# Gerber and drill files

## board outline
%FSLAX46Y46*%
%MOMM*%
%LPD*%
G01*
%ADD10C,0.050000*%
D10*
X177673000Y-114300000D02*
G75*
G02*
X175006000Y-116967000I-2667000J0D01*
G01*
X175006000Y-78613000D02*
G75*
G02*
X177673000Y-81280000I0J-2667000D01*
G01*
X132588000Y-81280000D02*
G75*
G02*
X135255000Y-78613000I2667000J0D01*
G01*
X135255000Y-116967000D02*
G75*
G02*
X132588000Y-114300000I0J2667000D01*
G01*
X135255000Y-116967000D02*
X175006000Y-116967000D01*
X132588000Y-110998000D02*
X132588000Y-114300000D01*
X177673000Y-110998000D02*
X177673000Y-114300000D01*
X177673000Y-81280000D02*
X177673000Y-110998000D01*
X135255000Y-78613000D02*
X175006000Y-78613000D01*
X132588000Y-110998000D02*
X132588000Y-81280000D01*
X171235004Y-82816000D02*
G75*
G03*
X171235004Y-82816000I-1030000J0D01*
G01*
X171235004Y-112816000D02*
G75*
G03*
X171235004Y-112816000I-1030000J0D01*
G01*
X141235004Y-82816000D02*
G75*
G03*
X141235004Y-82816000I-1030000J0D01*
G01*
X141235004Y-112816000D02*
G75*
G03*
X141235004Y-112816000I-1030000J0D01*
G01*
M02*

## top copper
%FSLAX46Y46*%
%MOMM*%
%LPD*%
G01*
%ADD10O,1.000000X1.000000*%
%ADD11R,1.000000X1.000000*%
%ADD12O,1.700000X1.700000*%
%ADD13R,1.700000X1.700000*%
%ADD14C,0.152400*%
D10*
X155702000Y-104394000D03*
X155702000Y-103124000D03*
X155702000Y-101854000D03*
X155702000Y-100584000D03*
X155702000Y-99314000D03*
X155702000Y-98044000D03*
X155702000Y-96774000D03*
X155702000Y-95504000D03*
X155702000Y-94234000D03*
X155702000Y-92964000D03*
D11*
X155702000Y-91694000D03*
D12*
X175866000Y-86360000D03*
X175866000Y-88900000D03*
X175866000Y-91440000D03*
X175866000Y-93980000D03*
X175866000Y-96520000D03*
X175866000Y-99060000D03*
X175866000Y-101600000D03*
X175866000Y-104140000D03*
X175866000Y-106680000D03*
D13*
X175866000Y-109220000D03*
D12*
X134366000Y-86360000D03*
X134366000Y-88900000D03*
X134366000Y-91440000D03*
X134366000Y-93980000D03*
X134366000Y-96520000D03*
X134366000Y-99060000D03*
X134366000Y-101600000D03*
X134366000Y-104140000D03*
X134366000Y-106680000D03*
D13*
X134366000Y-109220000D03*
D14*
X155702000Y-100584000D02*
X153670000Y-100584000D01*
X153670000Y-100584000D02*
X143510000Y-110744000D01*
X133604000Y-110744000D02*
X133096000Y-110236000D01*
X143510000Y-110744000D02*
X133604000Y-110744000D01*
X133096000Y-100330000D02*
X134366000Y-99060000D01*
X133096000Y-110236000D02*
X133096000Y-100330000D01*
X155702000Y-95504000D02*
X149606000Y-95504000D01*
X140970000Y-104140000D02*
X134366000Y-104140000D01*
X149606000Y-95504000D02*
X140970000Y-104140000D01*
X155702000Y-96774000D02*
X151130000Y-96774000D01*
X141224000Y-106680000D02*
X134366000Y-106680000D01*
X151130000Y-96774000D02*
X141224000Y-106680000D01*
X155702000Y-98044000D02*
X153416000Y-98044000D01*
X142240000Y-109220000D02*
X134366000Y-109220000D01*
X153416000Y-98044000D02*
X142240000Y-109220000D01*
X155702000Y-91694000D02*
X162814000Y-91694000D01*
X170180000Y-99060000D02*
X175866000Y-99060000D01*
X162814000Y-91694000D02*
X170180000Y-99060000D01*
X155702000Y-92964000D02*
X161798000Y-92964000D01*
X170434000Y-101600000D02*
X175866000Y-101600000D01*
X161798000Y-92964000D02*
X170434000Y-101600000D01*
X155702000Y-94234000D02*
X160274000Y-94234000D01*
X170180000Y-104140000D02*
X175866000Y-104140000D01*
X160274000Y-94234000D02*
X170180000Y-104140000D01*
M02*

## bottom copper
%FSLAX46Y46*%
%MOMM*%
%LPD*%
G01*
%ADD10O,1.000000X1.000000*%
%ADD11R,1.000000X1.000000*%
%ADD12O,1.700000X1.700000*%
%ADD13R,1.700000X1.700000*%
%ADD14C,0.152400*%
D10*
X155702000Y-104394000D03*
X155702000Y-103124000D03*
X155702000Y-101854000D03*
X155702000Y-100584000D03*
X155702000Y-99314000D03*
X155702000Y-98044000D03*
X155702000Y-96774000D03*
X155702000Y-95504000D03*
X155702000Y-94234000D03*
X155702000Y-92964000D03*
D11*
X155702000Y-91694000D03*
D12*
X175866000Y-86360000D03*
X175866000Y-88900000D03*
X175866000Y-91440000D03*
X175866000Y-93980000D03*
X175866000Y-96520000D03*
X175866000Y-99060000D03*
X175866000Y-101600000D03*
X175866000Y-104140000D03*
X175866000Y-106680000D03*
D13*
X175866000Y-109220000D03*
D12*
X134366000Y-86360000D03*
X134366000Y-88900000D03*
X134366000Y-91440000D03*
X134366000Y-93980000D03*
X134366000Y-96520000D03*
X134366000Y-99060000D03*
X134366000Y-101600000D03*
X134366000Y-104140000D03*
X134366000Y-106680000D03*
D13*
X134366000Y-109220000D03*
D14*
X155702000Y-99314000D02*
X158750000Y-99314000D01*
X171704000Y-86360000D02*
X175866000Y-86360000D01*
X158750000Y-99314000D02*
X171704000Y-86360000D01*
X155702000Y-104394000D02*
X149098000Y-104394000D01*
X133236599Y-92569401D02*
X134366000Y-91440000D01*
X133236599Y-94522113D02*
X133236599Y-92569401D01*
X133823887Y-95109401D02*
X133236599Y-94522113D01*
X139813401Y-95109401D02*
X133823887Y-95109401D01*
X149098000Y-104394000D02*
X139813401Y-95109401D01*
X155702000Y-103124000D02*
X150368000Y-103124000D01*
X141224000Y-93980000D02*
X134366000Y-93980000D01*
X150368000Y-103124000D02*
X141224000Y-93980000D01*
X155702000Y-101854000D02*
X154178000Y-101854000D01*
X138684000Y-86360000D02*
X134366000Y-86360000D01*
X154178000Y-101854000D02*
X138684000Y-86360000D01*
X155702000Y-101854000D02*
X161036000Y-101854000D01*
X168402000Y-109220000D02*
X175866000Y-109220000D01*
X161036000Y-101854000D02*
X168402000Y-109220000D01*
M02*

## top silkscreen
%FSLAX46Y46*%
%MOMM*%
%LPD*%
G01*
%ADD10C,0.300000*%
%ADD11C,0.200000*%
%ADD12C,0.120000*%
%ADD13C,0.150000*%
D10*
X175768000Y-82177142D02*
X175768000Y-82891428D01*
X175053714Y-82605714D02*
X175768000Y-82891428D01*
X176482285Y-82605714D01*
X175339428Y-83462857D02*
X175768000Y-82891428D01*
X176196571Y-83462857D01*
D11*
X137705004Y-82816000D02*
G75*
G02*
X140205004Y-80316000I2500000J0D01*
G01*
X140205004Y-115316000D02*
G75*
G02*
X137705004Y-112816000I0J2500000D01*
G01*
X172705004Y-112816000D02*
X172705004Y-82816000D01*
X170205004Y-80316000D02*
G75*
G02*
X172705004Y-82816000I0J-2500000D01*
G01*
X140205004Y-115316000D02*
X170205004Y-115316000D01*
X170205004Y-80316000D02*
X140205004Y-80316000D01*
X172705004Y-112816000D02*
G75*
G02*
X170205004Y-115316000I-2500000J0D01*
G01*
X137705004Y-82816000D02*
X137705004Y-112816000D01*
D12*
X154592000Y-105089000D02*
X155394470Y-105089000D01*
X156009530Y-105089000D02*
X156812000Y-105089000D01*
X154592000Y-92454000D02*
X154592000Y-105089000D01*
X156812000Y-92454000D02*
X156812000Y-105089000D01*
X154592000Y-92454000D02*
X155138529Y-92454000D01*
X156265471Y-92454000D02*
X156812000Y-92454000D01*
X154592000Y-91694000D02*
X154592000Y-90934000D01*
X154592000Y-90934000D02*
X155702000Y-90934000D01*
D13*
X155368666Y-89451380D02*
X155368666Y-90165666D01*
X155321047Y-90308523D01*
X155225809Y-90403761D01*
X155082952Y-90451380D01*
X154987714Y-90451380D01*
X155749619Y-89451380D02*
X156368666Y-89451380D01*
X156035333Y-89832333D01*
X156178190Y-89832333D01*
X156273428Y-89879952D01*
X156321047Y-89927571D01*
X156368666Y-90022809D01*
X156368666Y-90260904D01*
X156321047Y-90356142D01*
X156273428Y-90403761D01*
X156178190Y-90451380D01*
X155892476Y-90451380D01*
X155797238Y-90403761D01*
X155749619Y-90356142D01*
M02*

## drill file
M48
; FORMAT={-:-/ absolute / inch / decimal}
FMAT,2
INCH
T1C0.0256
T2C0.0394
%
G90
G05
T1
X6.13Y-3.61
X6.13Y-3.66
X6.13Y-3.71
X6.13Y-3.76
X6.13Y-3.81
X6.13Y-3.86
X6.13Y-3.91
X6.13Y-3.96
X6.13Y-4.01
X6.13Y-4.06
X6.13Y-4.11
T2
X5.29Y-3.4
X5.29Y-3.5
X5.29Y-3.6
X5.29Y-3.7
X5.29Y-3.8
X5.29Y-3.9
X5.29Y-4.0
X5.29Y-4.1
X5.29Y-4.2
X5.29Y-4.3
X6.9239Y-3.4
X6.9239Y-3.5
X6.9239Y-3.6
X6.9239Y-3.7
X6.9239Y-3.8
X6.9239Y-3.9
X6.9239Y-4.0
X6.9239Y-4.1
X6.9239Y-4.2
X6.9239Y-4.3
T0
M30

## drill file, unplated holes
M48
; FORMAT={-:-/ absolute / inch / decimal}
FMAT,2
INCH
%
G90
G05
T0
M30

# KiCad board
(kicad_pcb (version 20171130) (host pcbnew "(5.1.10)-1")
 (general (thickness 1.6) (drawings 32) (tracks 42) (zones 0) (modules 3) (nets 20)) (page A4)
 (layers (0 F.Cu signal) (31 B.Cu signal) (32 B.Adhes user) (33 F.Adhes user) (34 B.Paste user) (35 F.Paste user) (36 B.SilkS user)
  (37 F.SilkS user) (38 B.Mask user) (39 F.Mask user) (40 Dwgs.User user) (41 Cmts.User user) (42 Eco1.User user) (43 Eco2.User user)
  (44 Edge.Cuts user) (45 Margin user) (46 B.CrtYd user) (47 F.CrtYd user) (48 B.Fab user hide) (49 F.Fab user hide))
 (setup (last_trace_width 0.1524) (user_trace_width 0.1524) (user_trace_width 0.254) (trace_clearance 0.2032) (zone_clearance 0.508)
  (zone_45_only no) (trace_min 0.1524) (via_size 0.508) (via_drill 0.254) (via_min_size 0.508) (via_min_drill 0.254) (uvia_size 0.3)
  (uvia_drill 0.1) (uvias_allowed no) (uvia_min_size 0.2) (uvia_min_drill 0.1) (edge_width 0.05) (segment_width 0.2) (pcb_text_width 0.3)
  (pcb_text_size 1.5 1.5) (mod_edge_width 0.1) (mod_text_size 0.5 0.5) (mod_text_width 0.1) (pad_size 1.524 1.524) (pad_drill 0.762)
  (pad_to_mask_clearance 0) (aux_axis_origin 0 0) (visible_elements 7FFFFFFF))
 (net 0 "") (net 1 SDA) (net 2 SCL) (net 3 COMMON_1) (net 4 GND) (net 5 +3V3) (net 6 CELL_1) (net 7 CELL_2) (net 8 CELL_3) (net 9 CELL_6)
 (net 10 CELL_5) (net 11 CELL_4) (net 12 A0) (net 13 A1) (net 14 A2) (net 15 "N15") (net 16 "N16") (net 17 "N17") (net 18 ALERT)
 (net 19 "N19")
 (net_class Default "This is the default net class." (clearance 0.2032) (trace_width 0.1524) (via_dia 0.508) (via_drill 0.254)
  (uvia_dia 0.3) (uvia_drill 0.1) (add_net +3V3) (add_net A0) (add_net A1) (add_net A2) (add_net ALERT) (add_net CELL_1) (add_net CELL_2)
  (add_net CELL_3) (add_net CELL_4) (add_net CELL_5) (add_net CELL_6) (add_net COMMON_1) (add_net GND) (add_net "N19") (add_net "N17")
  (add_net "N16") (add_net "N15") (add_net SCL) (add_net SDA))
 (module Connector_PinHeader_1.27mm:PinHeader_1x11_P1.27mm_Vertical (layer F.Cu) (at 155.702 91.694)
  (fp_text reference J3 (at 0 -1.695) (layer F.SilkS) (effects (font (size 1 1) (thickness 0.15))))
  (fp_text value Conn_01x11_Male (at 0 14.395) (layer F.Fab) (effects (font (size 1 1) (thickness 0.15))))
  (fp_line (start -1.11 13.395) (end -0.30753 13.395) (layer F.SilkS) (width 0.12))
  (fp_line (start 0.30753 13.395) (end 1.11 13.395) (layer F.SilkS) (width 0.12))
  (fp_line (start -1.11 0.76) (end -1.11 13.395) (layer F.SilkS) (width 0.12))
  (fp_line (start 1.11 0.76) (end 1.11 13.395) (layer F.SilkS) (width 0.12))
  (fp_line (start -1.11 0.76) (end -0.563471 0.76) (layer F.SilkS) (width 0.12))
  (fp_line (start 0.563471 0.76) (end 1.11 0.76) (layer F.SilkS) (width 0.12))
  (fp_line (start -1.11 0) (end -1.11 -0.76) (layer F.SilkS) (width 0.12))
  (fp_line (start -1.11 -0.76) (end 0 -0.76) (layer F.SilkS) (width 0.12))
  (pad 11 thru_hole oval (at 0 12.7) (size 1 1) (drill 0.65) (layers *.Cu *.Mask) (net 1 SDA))
  (pad 10 thru_hole oval (at 0 11.43) (size 1 1) (drill 0.65) (layers *.Cu *.Mask) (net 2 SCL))
  (pad 9 thru_hole oval (at 0 10.16) (size 1 1) (drill 0.65) (layers *.Cu *.Mask) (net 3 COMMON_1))
  (pad 8 thru_hole oval (at 0 8.89) (size 1 1) (drill 0.65) (layers *.Cu *.Mask) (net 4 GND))
  (pad 7 thru_hole oval (at 0 7.62) (size 1 1) (drill 0.65) (layers *.Cu *.Mask) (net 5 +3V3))
  (pad 6 thru_hole oval (at 0 6.35) (size 1 1) (drill 0.65) (layers *.Cu *.Mask) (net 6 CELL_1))
  (pad 5 thru_hole oval (at 0 5.08) (size 1 1) (drill 0.65) (layers *.Cu *.Mask) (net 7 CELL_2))
  (pad 4 thru_hole oval (at 0 3.81) (size 1 1) (drill 0.65) (layers *.Cu *.Mask) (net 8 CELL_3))
  (pad 3 thru_hole oval (at 0 2.54) (size 1 1) (drill 0.65) (layers *.Cu *.Mask) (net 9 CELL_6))
  (pad 2 thru_hole oval (at 0 1.27) (size 1 1) (drill 0.65) (layers *.Cu *.Mask) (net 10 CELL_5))
  (pad 1 thru_hole rect (at 0 0) (size 1 1) (drill 0.65) (layers *.Cu *.Mask) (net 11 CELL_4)))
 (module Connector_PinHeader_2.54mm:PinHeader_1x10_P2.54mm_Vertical (layer B.Cu) (at 175.866 109.22)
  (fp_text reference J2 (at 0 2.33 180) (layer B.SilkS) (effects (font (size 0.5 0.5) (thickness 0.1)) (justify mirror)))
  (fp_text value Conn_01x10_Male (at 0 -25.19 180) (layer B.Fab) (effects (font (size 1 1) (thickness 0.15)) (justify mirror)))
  (pad 10 thru_hole oval (at 0 -22.86) (size 1.7 1.7) (drill 1) (layers *.Cu *.Mask) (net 5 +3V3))
  (pad 9 thru_hole oval (at 0 -20.32) (size 1.7 1.7) (drill 1) (layers *.Cu *.Mask) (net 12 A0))
  (pad 8 thru_hole oval (at 0 -17.78) (size 1.7 1.7) (drill 1) (layers *.Cu *.Mask) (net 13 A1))
  (pad 7 thru_hole oval (at 0 -15.24) (size 1.7 1.7) (drill 1) (layers *.Cu *.Mask) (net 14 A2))
  (pad 6 thru_hole oval (at 0 -12.7) (size 1.7 1.7) (drill 1) (layers *.Cu *.Mask) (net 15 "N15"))
  (pad 5 thru_hole oval (at 0 -10.16) (size 1.7 1.7) (drill 1) (layers *.Cu *.Mask) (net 11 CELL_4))
  (pad 4 thru_hole oval (at 0 -7.62) (size 1.7 1.7) (drill 1) (layers *.Cu *.Mask) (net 10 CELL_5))
  (pad 3 thru_hole oval (at 0 -5.08) (size 1.7 1.7) (drill 1) (layers *.Cu *.Mask) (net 9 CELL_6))
  (pad 2 thru_hole oval (at 0 -2.54) (size 1.7 1.7) (drill 1) (layers *.Cu *.Mask) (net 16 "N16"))
  (pad 1 thru_hole rect (at 0 0) (size 1.7 1.7) (drill 1) (layers *.Cu *.Mask) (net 3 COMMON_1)))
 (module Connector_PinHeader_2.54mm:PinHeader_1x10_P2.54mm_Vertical (layer B.Cu) (at 134.366 109.22)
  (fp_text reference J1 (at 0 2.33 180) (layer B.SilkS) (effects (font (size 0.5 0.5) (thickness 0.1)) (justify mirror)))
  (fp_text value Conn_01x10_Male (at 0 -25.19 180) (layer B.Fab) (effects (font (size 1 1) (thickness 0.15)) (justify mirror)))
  (pad 10 thru_hole oval (at 0 -22.86) (size 1.7 1.7) (drill 1) (layers *.Cu *.Mask) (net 3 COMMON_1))
  (pad 9 thru_hole oval (at 0 -20.32) (size 1.7 1.7) (drill 1) (layers *.Cu *.Mask) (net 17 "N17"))
  (pad 8 thru_hole oval (at 0 -17.78) (size 1.7 1.7) (drill 1) (layers *.Cu *.Mask) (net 1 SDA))
  (pad 7 thru_hole oval (at 0 -15.24) (size 1.7 1.7) (drill 1) (layers *.Cu *.Mask) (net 2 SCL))
  (pad 6 thru_hole oval (at 0 -12.7) (size 1.7 1.7) (drill 1) (layers *.Cu *.Mask) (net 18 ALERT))
  (pad 5 thru_hole oval (at 0 -10.16) (size 1.7 1.7) (drill 1) (layers *.Cu *.Mask) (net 4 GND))
  (pad 4 thru_hole oval (at 0 -7.62) (size 1.7 1.7) (drill 1) (layers *.Cu *.Mask) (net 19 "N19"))
  (pad 3 thru_hole oval (at 0 -5.08) (size 1.7 1.7) (drill 1) (layers *.Cu *.Mask) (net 8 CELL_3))
  (pad 2 thru_hole oval (at 0 -2.54) (size 1.7 1.7) (drill 1) (layers *.Cu *.Mask) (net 7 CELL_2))
  (pad 1 thru_hole rect (at 0 0) (size 1.7 1.7) (drill 1) (layers *.Cu *.Mask) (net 6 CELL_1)))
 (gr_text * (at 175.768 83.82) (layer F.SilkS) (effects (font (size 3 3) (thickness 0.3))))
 (gr_arc (start 175.006 114.3) (end 175.006 116.967) (angle -90) (layer Edge.Cuts) (width 0.05))
 (gr_arc (start 175.006 81.28) (end 177.673 81.28) (angle -90) (layer Edge.Cuts) (width 0.05))
 (gr_arc (start 135.255 81.28) (end 135.255 78.613) (angle -90) (layer Edge.Cuts) (width 0.05))
 (gr_arc (start 135.255 114.3) (end 132.588 114.3) (angle -90) (layer Edge.Cuts) (width 0.05))
 (gr_line (start 135.255 116.967) (end 175.006 116.967) (layer Edge.Cuts) (width 0.05))
 (gr_line (start 132.588 110.998) (end 132.588 114.3) (layer Edge.Cuts) (width 0.05))
 (gr_line (start 177.673 110.998) (end 177.673 114.3) (layer Edge.Cuts) (width 0.05))
 (gr_line (start 177.673 81.28) (end 177.673 110.998) (layer Edge.Cuts) (width 0.05))
 (gr_line (start 135.255 78.613) (end 175.006 78.613) (layer Edge.Cuts) (width 0.05))
 (gr_line (start 132.588 110.998) (end 132.588 81.28) (layer Edge.Cuts) (width 0.05))
 (gr_arc (start 140.205004 82.816) (end 140.205004 80.316) (angle -90) (layer F.SilkS) (width 0.2))
 (gr_circle (center 170.205004 82.816) (end 170.205004 81.786) (layer Edge.Cuts) (width 0.05))
 (gr_arc (start 140.205004 112.816) (end 137.705004 112.816) (angle -90) (layer F.SilkS) (width 0.2))
 (gr_line (start 172.705004 112.816) (end 172.705004 82.816) (layer F.SilkS) (width 0.2))
 (gr_arc (start 170.205004 82.816) (end 172.705004 82.816) (angle -90) (layer F.SilkS) (width 0.2))
 (gr_line (start 140.205004 115.316) (end 170.205004 115.316) (layer F.SilkS) (width 0.2))
 (gr_line (start 170.205004 80.316) (end 140.205004 80.316) (layer F.SilkS) (width 0.2))
 (gr_circle (center 170.205004 112.816) (end 170.205004 111.786) (layer Edge.Cuts) (width 0.05))
 (gr_arc (start 170.205004 112.816) (end 170.205004 115.316) (angle -90) (layer F.SilkS) (width 0.2))
 (gr_circle (center 140.205004 82.816) (end 140.205004 81.786) (layer Edge.Cuts) (width 0.05))
 (gr_circle (center 140.205004 112.816) (end 140.205004 111.786) (layer Edge.Cuts) (width 0.05))
 (gr_line (start 137.705004 82.816) (end 137.705004 112.816) (layer F.SilkS) (width 0.2))
 (segment (start 155.702 100.584) (end 153.67 100.584) (width 0.1524) (layer F.Cu) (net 4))
 (segment (start 153.67 100.584) (end 143.51 110.744) (width 0.1524) (layer F.Cu) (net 4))
 (segment (start 133.604 110.744) (end 133.096 110.236) (width 0.1524) (layer F.Cu) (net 4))
 (segment (start 143.51 110.744) (end 133.604 110.744) (width 0.1524) (layer F.Cu) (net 4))
 (segment (start 133.096 100.33) (end 134.366 99.06) (width 0.1524) (layer F.Cu) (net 4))
 (segment (start 133.096 110.236) (end 133.096 100.33) (width 0.1524) (layer F.Cu) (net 4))
 (segment (start 155.702 99.314) (end 158.75 99.314) (width 0.1524) (layer B.Cu) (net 5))
 (segment (start 171.704 86.36) (end 175.866 86.36) (width 0.1524) (layer B.Cu) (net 5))
 (segment (start 158.75 99.314) (end 171.704 86.36) (width 0.1524) (layer B.Cu) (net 5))
 (segment (start 155.702 104.394) (end 149.098 104.394) (width 0.1524) (layer B.Cu) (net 1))
 (segment (start 133.236599 92.569401) (end 134.366 91.44) (width 0.1524) (layer B.Cu) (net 1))
 (segment (start 133.236599 94.522113) (end 133.236599 92.569401) (width 0.1524) (layer B.Cu) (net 1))
 (segment (start 133.823887 95.109401) (end 133.236599 94.522113) (width 0.1524) (layer B.Cu) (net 1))
 (segment (start 139.813401 95.109401) (end 133.823887 95.109401) (width 0.1524) (layer B.Cu) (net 1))
 (segment (start 149.098 104.394) (end 139.813401 95.109401) (width 0.1524) (layer B.Cu) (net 1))
 (segment (start 155.702 103.124) (end 150.368 103.124) (width 0.1524) (layer B.Cu) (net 2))
 (segment (start 141.224 93.98) (end 134.366 93.98) (width 0.1524) (layer B.Cu) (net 2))
 (segment (start 150.368 103.124) (end 141.224 93.98) (width 0.1524) (layer B.Cu) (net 2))
 (segment (start 155.702 95.504) (end 149.606 95.504) (width 0.1524) (layer F.Cu) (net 8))
 (segment (start 140.97 104.14) (end 134.366 104.14) (width 0.1524) (layer F.Cu) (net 8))
 (segment (start 149.606 95.504) (end 140.97 104.14) (width 0.1524) (layer F.Cu) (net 8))
 (segment (start 155.702 96.774) (end 151.13 96.774) (width 0.1524) (layer F.Cu) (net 7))
 (segment (start 141.224 106.68) (end 134.366 106.68) (width 0.1524) (layer F.Cu) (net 7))
 (segment (start 151.13 96.774) (end 141.224 106.68) (width 0.1524) (layer F.Cu) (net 7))
 (segment (start 155.702 98.044) (end 153.416 98.044) (width 0.1524) (layer F.Cu) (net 6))
 (segment (start 142.24 109.22) (end 134.366 109.22) (width 0.1524) (layer F.Cu) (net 6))
 (segment (start 153.416 98.044) (end 142.24 109.22) (width 0.1524) (layer F.Cu) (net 6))
 (segment (start 155.702 91.694) (end 162.814 91.694) (width 0.1524) (layer F.Cu) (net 11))
 (segment (start 170.18 99.06) (end 175.866 99.06) (width 0.1524) (layer F.Cu) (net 11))
 (segment (start 162.814 91.694) (end 170.18 99.06) (width 0.1524) (layer F.Cu) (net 11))
 (segment (start 155.702 92.964) (end 161.798 92.964) (width 0.1524) (layer F.Cu) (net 10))
 (segment (start 170.434 101.6) (end 175.866 101.6) (width 0.1524) (layer F.Cu) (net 10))
 (segment (start 161.798 92.964) (end 170.434 101.6) (width 0.1524) (layer F.Cu) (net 10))
 (segment (start 155.702 94.234) (end 160.274 94.234) (width 0.1524) (layer F.Cu) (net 9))
 (segment (start 170.18 104.14) (end 175.866 104.14) (width 0.1524) (layer F.Cu) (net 9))
 (segment (start 160.274 94.234) (end 170.18 104.14) (width 0.1524) (layer F.Cu) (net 9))
 (segment (start 155.702 101.854) (end 154.178 101.854) (width 0.1524) (layer B.Cu) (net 3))
 (segment (start 138.684 86.36) (end 134.366 86.36) (width 0.1524) (layer B.Cu) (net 3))
 (segment (start 154.178 101.854) (end 138.684 86.36) (width 0.1524) (layer B.Cu) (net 3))
 (segment (start 155.702 101.854) (end 161.036 101.854) (width 0.1524) (layer B.Cu) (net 3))
 (segment (start 168.402 109.22) (end 175.866 109.22) (width 0.1524) (layer B.Cu) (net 3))
 (segment (start 161.036 101.854) (end 168.402 109.22) (width 0.1524) (layer B.Cu) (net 3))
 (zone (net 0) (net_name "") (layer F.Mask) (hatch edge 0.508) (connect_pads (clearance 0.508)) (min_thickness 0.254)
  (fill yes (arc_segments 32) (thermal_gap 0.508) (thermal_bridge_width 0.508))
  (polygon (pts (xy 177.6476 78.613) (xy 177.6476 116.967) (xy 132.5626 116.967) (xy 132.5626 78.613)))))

